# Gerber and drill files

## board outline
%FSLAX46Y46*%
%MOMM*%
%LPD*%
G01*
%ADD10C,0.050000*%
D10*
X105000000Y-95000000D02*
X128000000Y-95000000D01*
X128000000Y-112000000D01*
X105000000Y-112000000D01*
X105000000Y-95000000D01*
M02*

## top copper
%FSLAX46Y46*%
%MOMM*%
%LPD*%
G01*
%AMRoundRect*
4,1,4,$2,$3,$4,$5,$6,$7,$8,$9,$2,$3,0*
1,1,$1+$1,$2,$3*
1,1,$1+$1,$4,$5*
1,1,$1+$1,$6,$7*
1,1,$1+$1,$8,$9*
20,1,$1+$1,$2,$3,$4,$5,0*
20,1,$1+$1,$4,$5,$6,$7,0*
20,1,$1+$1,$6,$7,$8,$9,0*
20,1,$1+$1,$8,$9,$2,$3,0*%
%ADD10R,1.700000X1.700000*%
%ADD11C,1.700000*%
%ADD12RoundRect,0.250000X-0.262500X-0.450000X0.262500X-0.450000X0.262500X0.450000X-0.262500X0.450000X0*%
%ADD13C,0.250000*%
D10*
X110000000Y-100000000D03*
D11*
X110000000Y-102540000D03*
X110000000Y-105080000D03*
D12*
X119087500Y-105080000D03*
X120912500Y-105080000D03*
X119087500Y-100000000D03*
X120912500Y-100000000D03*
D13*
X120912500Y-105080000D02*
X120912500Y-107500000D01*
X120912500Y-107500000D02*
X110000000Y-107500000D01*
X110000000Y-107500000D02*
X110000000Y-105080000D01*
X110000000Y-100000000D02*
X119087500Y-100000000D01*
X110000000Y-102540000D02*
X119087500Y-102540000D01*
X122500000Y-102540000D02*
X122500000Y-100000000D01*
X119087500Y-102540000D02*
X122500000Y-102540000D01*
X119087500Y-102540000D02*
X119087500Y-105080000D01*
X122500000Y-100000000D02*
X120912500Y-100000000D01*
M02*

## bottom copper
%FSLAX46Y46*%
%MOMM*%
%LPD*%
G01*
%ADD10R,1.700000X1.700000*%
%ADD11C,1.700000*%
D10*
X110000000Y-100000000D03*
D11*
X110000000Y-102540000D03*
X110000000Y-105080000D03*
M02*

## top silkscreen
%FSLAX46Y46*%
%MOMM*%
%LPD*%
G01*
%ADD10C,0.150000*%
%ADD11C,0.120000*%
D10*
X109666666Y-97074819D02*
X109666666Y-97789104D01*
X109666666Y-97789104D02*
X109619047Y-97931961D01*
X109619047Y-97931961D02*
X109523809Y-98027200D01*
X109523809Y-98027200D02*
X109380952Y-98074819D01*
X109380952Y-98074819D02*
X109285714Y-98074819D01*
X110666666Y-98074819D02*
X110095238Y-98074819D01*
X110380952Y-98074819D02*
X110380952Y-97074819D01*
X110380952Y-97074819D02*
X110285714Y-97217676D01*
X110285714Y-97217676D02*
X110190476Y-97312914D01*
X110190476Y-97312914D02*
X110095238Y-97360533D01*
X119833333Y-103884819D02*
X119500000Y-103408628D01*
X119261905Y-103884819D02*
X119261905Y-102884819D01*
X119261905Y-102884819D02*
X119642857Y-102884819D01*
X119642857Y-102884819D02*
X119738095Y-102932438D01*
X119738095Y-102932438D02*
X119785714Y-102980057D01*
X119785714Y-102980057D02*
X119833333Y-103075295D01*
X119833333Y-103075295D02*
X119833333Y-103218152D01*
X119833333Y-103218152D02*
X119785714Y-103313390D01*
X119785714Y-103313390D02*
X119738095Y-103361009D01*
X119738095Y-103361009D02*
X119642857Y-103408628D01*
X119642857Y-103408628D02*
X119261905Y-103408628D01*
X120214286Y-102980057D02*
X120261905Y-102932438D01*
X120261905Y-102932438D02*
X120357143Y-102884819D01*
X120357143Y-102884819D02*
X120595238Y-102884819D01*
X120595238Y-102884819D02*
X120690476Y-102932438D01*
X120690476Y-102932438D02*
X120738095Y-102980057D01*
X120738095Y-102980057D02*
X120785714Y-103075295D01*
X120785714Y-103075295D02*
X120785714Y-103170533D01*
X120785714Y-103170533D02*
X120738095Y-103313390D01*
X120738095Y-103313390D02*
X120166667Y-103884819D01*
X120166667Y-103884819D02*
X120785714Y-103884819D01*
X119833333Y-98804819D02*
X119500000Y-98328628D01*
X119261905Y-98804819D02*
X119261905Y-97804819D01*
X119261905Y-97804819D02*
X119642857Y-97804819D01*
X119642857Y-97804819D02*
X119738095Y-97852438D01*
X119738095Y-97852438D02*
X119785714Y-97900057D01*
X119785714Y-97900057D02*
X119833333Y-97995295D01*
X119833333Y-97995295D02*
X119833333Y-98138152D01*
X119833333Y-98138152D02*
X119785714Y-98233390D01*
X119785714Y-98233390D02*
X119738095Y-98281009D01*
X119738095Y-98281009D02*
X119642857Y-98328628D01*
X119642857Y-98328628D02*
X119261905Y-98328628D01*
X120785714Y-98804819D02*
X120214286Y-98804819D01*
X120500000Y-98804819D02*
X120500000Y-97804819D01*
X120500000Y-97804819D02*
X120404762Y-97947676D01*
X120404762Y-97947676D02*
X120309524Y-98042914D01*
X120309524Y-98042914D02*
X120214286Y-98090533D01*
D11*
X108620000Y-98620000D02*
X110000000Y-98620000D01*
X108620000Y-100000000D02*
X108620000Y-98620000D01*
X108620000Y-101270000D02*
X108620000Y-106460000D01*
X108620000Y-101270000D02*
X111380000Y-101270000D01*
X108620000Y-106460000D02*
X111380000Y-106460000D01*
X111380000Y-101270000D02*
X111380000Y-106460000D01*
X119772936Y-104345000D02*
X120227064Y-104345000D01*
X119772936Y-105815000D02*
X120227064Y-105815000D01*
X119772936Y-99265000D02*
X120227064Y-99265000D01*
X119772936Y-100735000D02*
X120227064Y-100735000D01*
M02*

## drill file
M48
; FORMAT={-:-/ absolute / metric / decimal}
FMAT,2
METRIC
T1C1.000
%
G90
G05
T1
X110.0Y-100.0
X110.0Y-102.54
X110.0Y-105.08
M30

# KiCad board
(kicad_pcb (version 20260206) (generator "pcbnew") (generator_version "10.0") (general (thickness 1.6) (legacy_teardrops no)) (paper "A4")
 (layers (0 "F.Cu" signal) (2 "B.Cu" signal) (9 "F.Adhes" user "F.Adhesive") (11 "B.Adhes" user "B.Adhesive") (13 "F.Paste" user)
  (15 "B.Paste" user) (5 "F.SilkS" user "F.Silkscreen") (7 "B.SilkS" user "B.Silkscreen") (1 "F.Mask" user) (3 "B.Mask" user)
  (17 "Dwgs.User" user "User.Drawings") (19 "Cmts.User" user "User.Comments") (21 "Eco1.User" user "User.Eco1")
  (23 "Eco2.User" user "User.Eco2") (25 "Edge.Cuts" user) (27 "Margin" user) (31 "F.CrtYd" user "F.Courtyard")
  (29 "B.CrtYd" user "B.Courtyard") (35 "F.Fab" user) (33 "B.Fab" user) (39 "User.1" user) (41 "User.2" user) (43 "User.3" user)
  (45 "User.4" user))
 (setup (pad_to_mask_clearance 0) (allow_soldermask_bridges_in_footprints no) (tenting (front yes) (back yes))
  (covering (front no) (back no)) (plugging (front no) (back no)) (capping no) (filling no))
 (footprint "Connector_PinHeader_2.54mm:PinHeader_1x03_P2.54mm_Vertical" (layer "F.Cu") (at 110 100)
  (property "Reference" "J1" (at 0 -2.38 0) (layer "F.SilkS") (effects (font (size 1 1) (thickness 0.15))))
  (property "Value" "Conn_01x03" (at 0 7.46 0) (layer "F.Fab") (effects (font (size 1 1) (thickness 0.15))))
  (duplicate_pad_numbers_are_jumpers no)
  (fp_line (start -1.38 -1.38) (end 0 -1.38) (stroke (width 0.12) (type solid)) (layer "F.SilkS"))
  (fp_line (start -1.38 0) (end -1.38 -1.38) (stroke (width 0.12) (type solid)) (layer "F.SilkS"))
  (fp_line (start -1.38 1.27) (end -1.38 6.46) (stroke (width 0.12) (type solid)) (layer "F.SilkS"))
  (fp_line (start -1.38 1.27) (end 1.38 1.27) (stroke (width 0.12) (type solid)) (layer "F.SilkS"))
  (fp_line (start -1.38 6.46) (end 1.38 6.46) (stroke (width 0.12) (type solid)) (layer "F.SilkS"))
  (fp_line (start 1.38 1.27) (end 1.38 6.46) (stroke (width 0.12) (type solid)) (layer "F.SilkS"))
  (pad "1" thru_hole rect (at 0 0) (size 1.7 1.7) (drill 1) (layers "*.Cu" "*.Mask") (remove_unused_layers no) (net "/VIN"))
  (pad "2" thru_hole circle (at 0 2.54) (size 1.7 1.7) (drill 1) (layers "*.Cu" "*.Mask") (remove_unused_layers no) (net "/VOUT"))
  (pad "3" thru_hole circle (at 0 5.08) (size 1.7 1.7) (drill 1) (layers "*.Cu" "*.Mask") (remove_unused_layers no) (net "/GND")))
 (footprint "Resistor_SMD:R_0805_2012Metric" (layer "F.Cu") (at 120 105.08)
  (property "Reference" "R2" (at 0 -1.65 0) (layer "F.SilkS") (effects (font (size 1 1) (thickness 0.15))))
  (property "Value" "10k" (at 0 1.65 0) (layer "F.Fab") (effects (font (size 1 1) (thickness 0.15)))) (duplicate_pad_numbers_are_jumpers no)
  (fp_line (start -0.227064 -0.735) (end 0.227064 -0.735) (stroke (width 0.12) (type solid)) (layer "F.SilkS"))
  (fp_line (start -0.227064 0.735) (end 0.227064 0.735) (stroke (width 0.12) (type solid)) (layer "F.SilkS"))
  (pad "1" smd roundrect (at -0.9125 0) (size 1.025 1.4) (layers "F.Cu" "F.Mask" "F.Paste") (roundrect_rratio 0.243902) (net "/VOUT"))
  (pad "2" smd roundrect (at 0.9125 0) (size 1.025 1.4) (layers "F.Cu" "F.Mask" "F.Paste") (roundrect_rratio 0.243902) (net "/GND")))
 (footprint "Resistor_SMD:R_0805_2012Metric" (layer "F.Cu") (at 120 100)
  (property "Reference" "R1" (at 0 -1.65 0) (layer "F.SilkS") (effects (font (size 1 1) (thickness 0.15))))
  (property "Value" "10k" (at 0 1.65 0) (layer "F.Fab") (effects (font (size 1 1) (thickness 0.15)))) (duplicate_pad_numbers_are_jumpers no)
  (fp_line (start -0.227064 -0.735) (end 0.227064 -0.735) (stroke (width 0.12) (type solid)) (layer "F.SilkS"))
  (fp_line (start -0.227064 0.735) (end 0.227064 0.735) (stroke (width 0.12) (type solid)) (layer "F.SilkS"))
  (pad "1" smd roundrect (at -0.9125 0) (size 1.025 1.4) (layers "F.Cu" "F.Mask" "F.Paste") (roundrect_rratio 0.243902) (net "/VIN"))
  (pad "2" smd roundrect (at 0.9125 0) (size 1.025 1.4) (layers "F.Cu" "F.Mask" "F.Paste") (roundrect_rratio 0.243902) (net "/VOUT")))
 (gr_rect (start 105 95) (end 128 112) (stroke (width 0.05) (type default)) (fill no) (layer "Edge.Cuts"))
 (segment (start 120.9125 105.08) (end 120.9125 107.5) (width 0.25) (layer "F.Cu") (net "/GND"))
 (segment (start 120.9125 107.5) (end 110 107.5) (width 0.25) (layer "F.Cu") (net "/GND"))
 (segment (start 110 107.5) (end 110 105.08) (width 0.25) (layer "F.Cu") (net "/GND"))
 (segment (start 110 100) (end 119.0875 100) (width 0.25) (layer "F.Cu") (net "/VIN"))
 (segment (start 110 102.54) (end 119.0875 102.54) (width 0.25) (layer "F.Cu") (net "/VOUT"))
 (segment (start 122.5 102.54) (end 122.5 100) (width 0.25) (layer "F.Cu") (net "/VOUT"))
 (segment (start 119.0875 102.54) (end 122.5 102.54) (width 0.25) (layer "F.Cu") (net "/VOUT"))
 (segment (start 119.0875 102.54) (end 119.0875 105.08) (width 0.25) (layer "F.Cu") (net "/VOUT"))
 (segment (start 122.5 100) (end 120.9125 100) (width 0.25) (layer "F.Cu") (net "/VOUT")))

